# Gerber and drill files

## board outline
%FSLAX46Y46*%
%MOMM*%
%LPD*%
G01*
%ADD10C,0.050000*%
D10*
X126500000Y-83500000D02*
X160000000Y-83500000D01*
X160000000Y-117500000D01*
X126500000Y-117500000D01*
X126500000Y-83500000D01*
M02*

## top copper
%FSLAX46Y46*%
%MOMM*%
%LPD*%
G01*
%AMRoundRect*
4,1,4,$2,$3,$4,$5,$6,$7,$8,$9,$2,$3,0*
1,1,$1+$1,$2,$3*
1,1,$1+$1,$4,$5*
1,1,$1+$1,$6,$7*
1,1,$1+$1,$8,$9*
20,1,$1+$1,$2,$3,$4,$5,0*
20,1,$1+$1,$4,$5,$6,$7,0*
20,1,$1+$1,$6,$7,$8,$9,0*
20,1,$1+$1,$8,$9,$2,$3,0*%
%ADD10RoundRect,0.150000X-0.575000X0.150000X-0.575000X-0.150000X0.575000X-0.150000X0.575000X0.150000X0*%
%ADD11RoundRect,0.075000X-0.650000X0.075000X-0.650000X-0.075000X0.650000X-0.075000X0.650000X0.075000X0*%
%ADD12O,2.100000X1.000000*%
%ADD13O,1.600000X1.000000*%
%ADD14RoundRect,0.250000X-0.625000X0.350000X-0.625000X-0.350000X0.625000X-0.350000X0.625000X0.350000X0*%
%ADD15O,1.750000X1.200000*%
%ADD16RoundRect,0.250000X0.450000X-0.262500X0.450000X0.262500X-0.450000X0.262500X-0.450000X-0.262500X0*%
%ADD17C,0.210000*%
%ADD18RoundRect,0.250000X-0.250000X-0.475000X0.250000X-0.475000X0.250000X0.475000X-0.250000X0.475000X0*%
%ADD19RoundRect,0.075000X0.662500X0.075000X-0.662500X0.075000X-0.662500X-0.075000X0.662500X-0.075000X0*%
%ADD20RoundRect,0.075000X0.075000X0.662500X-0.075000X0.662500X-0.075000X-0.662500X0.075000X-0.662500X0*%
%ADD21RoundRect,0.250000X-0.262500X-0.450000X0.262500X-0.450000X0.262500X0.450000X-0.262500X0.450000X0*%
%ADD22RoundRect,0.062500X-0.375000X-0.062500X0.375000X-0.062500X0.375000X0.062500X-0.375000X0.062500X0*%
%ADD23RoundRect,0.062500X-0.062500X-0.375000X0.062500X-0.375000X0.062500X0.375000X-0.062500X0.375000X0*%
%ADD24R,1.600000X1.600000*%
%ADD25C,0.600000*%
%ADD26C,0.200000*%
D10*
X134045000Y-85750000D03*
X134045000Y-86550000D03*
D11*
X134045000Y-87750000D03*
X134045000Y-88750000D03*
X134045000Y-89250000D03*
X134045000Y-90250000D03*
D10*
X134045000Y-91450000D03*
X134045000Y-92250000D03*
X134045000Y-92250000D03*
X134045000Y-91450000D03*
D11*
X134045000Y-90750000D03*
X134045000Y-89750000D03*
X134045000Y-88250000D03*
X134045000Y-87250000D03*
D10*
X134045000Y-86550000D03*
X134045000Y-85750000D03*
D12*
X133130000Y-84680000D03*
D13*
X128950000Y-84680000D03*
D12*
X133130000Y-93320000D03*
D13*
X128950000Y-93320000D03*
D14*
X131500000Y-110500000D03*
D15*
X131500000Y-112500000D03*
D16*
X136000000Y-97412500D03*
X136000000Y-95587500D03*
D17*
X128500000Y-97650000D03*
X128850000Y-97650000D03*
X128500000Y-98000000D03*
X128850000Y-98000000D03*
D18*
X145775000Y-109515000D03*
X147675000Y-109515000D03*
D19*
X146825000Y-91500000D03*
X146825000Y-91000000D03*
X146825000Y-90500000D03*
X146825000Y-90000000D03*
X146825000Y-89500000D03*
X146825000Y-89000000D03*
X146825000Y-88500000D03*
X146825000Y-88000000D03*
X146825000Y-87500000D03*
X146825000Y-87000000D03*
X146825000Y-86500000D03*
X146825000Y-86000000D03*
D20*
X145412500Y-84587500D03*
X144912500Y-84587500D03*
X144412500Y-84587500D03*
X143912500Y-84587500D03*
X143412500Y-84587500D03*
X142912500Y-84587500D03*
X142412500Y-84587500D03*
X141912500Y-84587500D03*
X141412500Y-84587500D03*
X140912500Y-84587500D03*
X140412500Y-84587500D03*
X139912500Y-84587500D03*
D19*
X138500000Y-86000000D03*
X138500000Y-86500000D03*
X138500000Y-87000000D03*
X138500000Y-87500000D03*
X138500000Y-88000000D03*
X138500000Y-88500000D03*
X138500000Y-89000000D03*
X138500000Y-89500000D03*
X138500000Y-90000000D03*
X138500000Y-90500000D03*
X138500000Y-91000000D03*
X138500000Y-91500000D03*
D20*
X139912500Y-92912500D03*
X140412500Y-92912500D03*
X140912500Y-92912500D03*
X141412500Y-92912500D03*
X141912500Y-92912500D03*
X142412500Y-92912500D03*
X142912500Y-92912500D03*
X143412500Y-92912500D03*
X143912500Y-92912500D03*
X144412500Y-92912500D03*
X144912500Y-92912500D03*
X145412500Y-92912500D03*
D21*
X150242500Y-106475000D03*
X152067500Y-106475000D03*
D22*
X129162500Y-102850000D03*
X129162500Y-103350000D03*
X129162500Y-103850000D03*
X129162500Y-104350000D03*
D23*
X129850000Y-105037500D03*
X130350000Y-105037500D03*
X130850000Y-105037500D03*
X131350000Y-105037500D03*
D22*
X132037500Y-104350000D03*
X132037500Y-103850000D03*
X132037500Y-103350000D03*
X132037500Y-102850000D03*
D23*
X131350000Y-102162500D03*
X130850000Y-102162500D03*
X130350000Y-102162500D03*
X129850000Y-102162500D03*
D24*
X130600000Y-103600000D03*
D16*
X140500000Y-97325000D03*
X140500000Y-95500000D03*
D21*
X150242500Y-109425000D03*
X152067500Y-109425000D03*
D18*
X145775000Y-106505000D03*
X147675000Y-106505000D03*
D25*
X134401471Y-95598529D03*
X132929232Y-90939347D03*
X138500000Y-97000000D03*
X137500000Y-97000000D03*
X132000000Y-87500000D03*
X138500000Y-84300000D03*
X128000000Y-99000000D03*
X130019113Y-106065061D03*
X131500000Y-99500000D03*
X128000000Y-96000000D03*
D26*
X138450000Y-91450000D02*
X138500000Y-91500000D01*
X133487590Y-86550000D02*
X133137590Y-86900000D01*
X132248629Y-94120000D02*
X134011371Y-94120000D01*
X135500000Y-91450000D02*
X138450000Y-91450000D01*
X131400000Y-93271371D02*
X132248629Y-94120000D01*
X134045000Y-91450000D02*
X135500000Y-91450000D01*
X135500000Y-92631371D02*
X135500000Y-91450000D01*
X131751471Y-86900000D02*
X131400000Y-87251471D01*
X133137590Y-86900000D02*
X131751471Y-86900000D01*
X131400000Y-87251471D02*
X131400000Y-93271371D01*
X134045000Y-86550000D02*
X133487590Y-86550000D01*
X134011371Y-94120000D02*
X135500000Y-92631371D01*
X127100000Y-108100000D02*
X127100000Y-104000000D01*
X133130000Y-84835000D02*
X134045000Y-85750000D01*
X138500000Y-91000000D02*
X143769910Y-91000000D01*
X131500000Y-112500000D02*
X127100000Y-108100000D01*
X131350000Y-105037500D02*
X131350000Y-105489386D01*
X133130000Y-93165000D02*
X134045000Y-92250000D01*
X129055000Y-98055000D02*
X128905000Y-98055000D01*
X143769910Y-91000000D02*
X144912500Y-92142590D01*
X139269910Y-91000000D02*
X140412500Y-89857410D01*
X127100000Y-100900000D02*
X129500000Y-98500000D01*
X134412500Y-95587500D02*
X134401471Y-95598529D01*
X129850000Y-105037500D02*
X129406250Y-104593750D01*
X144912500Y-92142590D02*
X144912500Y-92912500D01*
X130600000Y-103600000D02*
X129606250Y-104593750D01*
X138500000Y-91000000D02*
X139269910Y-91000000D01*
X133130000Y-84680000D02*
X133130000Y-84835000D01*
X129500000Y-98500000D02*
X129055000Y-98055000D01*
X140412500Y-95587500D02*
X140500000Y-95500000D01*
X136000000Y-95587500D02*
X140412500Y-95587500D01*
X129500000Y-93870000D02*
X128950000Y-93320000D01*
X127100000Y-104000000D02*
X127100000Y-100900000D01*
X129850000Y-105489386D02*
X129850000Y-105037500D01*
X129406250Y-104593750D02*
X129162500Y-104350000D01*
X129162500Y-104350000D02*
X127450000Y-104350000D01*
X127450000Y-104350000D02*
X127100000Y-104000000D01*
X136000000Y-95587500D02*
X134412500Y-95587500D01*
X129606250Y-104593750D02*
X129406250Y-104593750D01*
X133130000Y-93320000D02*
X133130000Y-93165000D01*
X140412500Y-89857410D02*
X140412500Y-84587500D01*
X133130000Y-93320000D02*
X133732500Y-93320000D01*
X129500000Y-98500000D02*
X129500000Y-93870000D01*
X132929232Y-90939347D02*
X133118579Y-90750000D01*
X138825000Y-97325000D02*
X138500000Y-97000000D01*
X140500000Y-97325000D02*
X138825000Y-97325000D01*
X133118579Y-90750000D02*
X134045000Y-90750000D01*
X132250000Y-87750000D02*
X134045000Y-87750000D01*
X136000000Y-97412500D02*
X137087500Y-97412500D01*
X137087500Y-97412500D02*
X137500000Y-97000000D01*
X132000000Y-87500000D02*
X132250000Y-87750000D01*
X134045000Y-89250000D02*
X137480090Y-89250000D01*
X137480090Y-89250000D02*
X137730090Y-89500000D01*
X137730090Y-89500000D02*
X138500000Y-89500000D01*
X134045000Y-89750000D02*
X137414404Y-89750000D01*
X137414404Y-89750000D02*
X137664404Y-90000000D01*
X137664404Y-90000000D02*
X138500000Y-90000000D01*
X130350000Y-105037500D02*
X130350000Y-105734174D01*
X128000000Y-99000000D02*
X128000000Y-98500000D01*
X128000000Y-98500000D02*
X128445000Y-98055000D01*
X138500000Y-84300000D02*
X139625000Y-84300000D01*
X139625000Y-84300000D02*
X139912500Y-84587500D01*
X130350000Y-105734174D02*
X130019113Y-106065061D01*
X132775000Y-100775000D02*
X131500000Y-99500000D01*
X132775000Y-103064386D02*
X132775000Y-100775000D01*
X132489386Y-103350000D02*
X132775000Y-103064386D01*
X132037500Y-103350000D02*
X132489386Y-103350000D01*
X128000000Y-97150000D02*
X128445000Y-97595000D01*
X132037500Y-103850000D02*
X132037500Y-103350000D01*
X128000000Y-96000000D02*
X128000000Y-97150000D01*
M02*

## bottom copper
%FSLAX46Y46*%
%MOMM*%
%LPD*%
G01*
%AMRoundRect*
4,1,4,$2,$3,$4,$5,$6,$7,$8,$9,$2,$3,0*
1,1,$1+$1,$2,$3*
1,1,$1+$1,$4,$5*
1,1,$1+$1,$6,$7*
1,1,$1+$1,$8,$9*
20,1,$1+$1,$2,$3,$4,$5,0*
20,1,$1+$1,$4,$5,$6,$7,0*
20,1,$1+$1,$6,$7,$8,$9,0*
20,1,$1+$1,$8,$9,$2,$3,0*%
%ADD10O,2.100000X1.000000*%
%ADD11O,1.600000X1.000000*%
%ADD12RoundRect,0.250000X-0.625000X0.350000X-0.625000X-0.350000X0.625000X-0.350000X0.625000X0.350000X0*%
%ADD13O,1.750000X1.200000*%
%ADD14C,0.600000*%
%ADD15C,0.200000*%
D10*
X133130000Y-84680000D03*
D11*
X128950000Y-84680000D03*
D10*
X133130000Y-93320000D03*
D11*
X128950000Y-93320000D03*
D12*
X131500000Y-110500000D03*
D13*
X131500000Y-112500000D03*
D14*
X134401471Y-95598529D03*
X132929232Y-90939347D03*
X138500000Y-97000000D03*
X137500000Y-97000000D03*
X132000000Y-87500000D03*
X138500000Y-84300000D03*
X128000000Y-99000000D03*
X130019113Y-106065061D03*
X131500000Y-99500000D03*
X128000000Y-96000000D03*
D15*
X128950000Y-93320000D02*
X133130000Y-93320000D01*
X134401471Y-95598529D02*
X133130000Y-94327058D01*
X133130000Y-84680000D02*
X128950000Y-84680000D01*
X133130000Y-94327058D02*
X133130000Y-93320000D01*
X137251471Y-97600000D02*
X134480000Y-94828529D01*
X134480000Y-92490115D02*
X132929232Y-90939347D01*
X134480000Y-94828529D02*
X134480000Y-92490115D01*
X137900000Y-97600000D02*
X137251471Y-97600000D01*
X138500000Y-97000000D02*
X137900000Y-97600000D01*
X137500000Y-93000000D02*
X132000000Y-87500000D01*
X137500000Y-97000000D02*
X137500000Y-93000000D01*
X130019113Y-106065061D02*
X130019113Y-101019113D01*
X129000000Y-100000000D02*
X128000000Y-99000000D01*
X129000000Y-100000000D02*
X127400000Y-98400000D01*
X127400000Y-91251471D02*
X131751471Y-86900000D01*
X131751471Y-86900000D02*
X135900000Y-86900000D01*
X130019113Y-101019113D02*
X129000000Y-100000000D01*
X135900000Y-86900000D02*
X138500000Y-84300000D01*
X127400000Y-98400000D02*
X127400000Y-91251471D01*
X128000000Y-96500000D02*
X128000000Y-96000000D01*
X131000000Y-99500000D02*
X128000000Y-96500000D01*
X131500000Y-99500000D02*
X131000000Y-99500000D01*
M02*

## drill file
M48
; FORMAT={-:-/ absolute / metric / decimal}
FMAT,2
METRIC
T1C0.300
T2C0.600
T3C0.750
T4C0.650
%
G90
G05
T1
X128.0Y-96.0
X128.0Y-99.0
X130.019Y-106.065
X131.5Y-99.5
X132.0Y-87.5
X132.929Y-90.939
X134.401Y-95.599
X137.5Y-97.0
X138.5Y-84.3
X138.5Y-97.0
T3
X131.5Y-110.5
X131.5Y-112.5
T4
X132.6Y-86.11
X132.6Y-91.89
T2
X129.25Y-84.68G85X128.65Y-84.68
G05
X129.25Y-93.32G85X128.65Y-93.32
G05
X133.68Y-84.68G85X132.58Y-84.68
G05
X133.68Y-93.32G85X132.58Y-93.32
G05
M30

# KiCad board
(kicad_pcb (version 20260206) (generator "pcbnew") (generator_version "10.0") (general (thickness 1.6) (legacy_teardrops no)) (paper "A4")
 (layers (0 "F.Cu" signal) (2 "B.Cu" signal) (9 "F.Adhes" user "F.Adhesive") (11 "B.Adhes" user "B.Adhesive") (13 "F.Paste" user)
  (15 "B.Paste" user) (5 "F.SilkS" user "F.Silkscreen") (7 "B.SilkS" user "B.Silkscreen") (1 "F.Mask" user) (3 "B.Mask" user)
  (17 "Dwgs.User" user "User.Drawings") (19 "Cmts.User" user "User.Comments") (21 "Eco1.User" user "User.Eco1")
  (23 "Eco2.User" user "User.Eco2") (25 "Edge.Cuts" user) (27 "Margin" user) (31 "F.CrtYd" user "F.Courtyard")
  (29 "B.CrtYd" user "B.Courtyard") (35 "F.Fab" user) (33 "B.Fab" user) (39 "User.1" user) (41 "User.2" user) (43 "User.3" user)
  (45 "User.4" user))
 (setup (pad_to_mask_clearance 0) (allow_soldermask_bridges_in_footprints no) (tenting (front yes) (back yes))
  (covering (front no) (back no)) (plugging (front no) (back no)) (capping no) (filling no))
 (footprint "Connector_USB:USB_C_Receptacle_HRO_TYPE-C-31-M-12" (layer "F.Cu") (at 130 89 -90)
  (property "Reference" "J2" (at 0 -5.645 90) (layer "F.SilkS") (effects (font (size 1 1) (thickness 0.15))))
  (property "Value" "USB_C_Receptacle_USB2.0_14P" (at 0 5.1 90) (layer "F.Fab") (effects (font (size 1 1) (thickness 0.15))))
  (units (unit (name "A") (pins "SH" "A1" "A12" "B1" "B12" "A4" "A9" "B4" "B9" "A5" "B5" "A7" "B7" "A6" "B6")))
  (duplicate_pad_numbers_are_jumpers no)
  (pad "" np_thru_hole circle (at -2.89 -2.6 270) (size 0.65 0.65) (drill 0.65) (layers "*.Cu" "*.Mask"))
  (pad "" np_thru_hole circle (at 2.89 -2.6 270) (size 0.65 0.65) (drill 0.65) (layers "*.Cu" "*.Mask"))
  (pad "A1" smd roundrect (at -3.25 -4.045 270) (size 0.6 1.45) (layers "F.Cu" "F.Mask" "F.Paste") (roundrect_rratio 0.25) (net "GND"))
  (pad "A4" smd roundrect (at -2.45 -4.045 270) (size 0.6 1.45) (layers "F.Cu" "F.Mask" "F.Paste") (roundrect_rratio 0.25)
   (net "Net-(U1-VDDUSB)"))
  (pad "A5" smd roundrect (at -1.25 -4.045 270) (size 0.3 1.45) (layers "F.Cu" "F.Mask" "F.Paste") (roundrect_rratio 0.25)
   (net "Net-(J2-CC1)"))
  (pad "A6" smd roundrect (at -0.25 -4.045 270) (size 0.3 1.45) (layers "F.Cu" "F.Mask" "F.Paste") (roundrect_rratio 0.25)
   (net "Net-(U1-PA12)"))
  (pad "A7" smd roundrect (at 0.25 -4.045 270) (size 0.3 1.45) (layers "F.Cu" "F.Mask" "F.Paste") (roundrect_rratio 0.25)
   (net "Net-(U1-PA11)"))
  (pad "A8" smd roundrect (at 1.25 -4.045 270) (size 0.3 1.45) (layers "F.Cu" "F.Mask" "F.Paste") (roundrect_rratio 0.25))
  (pad "A9" smd roundrect (at 2.45 -4.045 270) (size 0.6 1.45) (layers "F.Cu" "F.Mask" "F.Paste") (roundrect_rratio 0.25)
   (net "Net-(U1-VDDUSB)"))
  (pad "A12" smd roundrect (at 3.25 -4.045 270) (size 0.6 1.45) (layers "F.Cu" "F.Mask" "F.Paste") (roundrect_rratio 0.25) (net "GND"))
  (pad "B1" smd roundrect (at 3.25 -4.045 270) (size 0.6 1.45) (layers "F.Cu" "F.Mask" "F.Paste") (roundrect_rratio 0.25) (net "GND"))
  (pad "B4" smd roundrect (at 2.45 -4.045 270) (size 0.6 1.45) (layers "F.Cu" "F.Mask" "F.Paste") (roundrect_rratio 0.25)
   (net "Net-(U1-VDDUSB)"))
  (pad "B5" smd roundrect (at 1.75 -4.045 270) (size 0.3 1.45) (layers "F.Cu" "F.Mask" "F.Paste") (roundrect_rratio 0.25)
   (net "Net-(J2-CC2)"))
  (pad "B6" smd roundrect (at 0.75 -4.045 270) (size 0.3 1.45) (layers "F.Cu" "F.Mask" "F.Paste") (roundrect_rratio 0.25)
   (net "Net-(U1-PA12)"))
  (pad "B7" smd roundrect (at -0.75 -4.045 270) (size 0.3 1.45) (layers "F.Cu" "F.Mask" "F.Paste") (roundrect_rratio 0.25)
   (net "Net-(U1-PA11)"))
  (pad "B8" smd roundrect (at -1.75 -4.045 270) (size 0.3 1.45) (layers "F.Cu" "F.Mask" "F.Paste") (roundrect_rratio 0.25))
  (pad "B9" smd roundrect (at -2.45 -4.045 270) (size 0.6 1.45) (layers "F.Cu" "F.Mask" "F.Paste") (roundrect_rratio 0.25)
   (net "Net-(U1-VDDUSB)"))
  (pad "B12" smd roundrect (at -3.25 -4.045 270) (size 0.6 1.45) (layers "F.Cu" "F.Mask" "F.Paste") (roundrect_rratio 0.25) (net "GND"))
  (pad "SH" thru_hole oval (at -4.32 -3.13 270) (size 1 2.1) (drill oval 0.6 1.7) (layers "*.Cu" "*.Mask") (remove_unused_layers no)
   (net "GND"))
  (pad "SH" thru_hole oval (at -4.32 1.05 270) (size 1 1.6) (drill oval 0.6 1.2) (layers "*.Cu" "*.Mask") (remove_unused_layers no)
   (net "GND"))
  (pad "SH" thru_hole oval (at 4.32 -3.13 270) (size 1 2.1) (drill oval 0.6 1.7) (layers "*.Cu" "*.Mask") (remove_unused_layers no)
   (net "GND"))
  (pad "SH" thru_hole oval (at 4.32 1.05 270) (size 1 1.6) (drill oval 0.6 1.2) (layers "*.Cu" "*.Mask") (remove_unused_layers no)
   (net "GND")))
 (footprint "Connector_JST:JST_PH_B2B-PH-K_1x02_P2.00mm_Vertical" (layer "F.Cu") (at 131.5 110.5 -90)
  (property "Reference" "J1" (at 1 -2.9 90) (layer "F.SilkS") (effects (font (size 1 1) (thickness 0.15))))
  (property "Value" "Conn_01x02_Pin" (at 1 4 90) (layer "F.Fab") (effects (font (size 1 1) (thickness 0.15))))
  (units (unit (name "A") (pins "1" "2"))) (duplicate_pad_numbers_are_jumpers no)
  (pad "1" thru_hole roundrect (at 0 0 270) (size 1.2 1.75) (drill 0.75) (layers "*.Cu" "*.Mask") (remove_unused_layers no)
   (roundrect_rratio 0.208333) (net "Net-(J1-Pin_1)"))
  (pad "2" thru_hole oval (at 2 0 270) (size 1.2 1.75) (drill 0.75) (layers "*.Cu" "*.Mask") (remove_unused_layers no) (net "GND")))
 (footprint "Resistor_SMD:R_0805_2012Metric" (layer "F.Cu") (at 136 96.5 90)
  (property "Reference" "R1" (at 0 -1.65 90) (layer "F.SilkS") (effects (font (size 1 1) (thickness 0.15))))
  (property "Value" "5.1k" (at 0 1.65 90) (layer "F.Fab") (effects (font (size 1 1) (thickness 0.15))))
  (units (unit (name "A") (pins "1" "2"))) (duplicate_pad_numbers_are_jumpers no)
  (pad "1" smd roundrect (at -0.9125 0 90) (size 1.025 1.4) (layers "F.Cu" "F.Mask" "F.Paste") (roundrect_rratio 0.243902)
   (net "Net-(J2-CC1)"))
  (pad "2" smd roundrect (at 0.9125 0 90) (size 1.025 1.4) (layers "F.Cu" "F.Mask" "F.Paste") (roundrect_rratio 0.243902) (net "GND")))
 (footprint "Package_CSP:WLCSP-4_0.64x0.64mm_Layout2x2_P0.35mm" (layer "F.Cu") (at 128.675 97.825)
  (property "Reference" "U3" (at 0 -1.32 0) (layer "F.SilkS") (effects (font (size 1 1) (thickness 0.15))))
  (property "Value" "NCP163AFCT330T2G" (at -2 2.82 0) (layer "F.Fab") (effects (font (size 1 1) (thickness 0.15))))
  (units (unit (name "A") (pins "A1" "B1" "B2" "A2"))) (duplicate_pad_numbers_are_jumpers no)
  (pad "A1" smd circle (at -0.175 -0.175) (size 0.21 0.21) (layers "F.Cu" "F.Mask" "F.Paste") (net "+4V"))
  (pad "A2" smd circle (at 0.175 -0.175) (size 0.21 0.21) (layers "F.Cu" "F.Mask" "F.Paste") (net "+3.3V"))
  (pad "B1" smd circle (at -0.175 0.175) (size 0.21 0.21) (layers "F.Cu" "F.Mask" "F.Paste") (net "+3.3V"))
  (pad "B2" smd circle (at 0.175 0.175) (size 0.21 0.21) (layers "F.Cu" "F.Mask" "F.Paste") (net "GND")))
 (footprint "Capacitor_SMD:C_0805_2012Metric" (layer "F.Cu") (at 146.725 109.515)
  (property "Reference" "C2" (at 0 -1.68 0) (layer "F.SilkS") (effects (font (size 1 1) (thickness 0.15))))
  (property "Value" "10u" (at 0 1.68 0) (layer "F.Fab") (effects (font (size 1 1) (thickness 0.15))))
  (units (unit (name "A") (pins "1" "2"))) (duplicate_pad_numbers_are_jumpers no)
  (pad "1" smd roundrect (at -0.95 0) (size 1 1.45) (layers "F.Cu" "F.Mask" "F.Paste") (roundrect_rratio 0.25) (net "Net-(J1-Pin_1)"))
  (pad "2" smd roundrect (at 0.95 0) (size 1 1.45) (layers "F.Cu" "F.Mask" "F.Paste") (roundrect_rratio 0.25) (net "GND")))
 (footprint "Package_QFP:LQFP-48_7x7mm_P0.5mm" (layer "F.Cu") (at 142.6625 88.75 180)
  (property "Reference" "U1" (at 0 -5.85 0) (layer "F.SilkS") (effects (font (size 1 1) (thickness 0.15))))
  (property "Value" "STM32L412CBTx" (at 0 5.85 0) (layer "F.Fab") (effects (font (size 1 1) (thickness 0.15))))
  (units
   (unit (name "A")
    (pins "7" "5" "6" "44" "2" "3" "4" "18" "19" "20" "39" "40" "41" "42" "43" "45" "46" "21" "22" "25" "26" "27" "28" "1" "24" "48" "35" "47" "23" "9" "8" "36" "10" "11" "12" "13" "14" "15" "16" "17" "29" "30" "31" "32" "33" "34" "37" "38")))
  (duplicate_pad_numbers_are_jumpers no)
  (pad "1" smd roundrect (at -4.1625 -2.75 180) (size 1.475 0.3) (layers "F.Cu" "F.Mask" "F.Paste") (roundrect_rratio 0.25) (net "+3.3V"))
  (pad "2" smd roundrect (at -4.1625 -2.25 180) (size 1.475 0.3) (layers "F.Cu" "F.Mask" "F.Paste") (roundrect_rratio 0.25)
   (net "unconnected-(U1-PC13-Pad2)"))
  (pad "3" smd roundrect (at -4.1625 -1.75 180) (size 1.475 0.3) (layers "F.Cu" "F.Mask" "F.Paste") (roundrect_rratio 0.25)
   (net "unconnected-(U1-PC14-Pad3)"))
  (pad "4" smd roundrect (at -4.1625 -1.25 180) (size 1.475 0.3) (layers "F.Cu" "F.Mask" "F.Paste") (roundrect_rratio 0.25)
   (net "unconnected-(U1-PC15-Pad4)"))
  (pad "5" smd roundrect (at -4.1625 -0.75 180) (size 1.475 0.3) (layers "F.Cu" "F.Mask" "F.Paste") (roundrect_rratio 0.25)
   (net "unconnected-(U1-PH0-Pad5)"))
  (pad "6" smd roundrect (at -4.1625 -0.25 180) (size 1.475 0.3) (layers "F.Cu" "F.Mask" "F.Paste") (roundrect_rratio 0.25)
   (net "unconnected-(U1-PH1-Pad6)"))
  (pad "7" smd roundrect (at -4.1625 0.25 180) (size 1.475 0.3) (layers "F.Cu" "F.Mask" "F.Paste") (roundrect_rratio 0.25)
   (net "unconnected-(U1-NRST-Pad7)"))
  (pad "8" smd roundrect (at -4.1625 0.75 180) (size 1.475 0.3) (layers "F.Cu" "F.Mask" "F.Paste") (roundrect_rratio 0.25) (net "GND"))
  (pad "9" smd roundrect (at -4.1625 1.25 180) (size 1.475 0.3) (layers "F.Cu" "F.Mask" "F.Paste") (roundrect_rratio 0.25) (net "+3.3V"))
  (pad "10" smd roundrect (at -4.1625 1.75 180) (size 1.475 0.3) (layers "F.Cu" "F.Mask" "F.Paste") (roundrect_rratio 0.25)
   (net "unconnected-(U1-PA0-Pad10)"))
  (pad "11" smd roundrect (at -4.1625 2.25 180) (size 1.475 0.3) (layers "F.Cu" "F.Mask" "F.Paste") (roundrect_rratio 0.25)
   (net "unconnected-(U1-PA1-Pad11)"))
  (pad "12" smd roundrect (at -4.1625 2.75 180) (size 1.475 0.3) (layers "F.Cu" "F.Mask" "F.Paste") (roundrect_rratio 0.25)
   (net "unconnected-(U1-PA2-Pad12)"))
  (pad "13" smd roundrect (at -2.75 4.1625 180) (size 0.3 1.475) (layers "F.Cu" "F.Mask" "F.Paste") (roundrect_rratio 0.25)
   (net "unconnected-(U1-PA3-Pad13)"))
  (pad "14" smd roundrect (at -2.25 4.1625 180) (size 0.3 1.475) (layers "F.Cu" "F.Mask" "F.Paste") (roundrect_rratio 0.25)
   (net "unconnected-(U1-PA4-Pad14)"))
  (pad "15" smd roundrect (at -1.75 4.1625 180) (size 0.3 1.475) (layers "F.Cu" "F.Mask" "F.Paste") (roundrect_rratio 0.25)
   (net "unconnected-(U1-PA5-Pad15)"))
  (pad "16" smd roundrect (at -1.25 4.1625 180) (size 0.3 1.475) (layers "F.Cu" "F.Mask" "F.Paste") (roundrect_rratio 0.25)
   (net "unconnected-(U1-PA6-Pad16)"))
  (pad "17" smd roundrect (at -0.75 4.1625 180) (size 0.3 1.475) (layers "F.Cu" "F.Mask" "F.Paste") (roundrect_rratio 0.25)
   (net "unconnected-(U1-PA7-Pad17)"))
  (pad "18" smd roundrect (at -0.25 4.1625 180) (size 0.3 1.475) (layers "F.Cu" "F.Mask" "F.Paste") (roundrect_rratio 0.25)
   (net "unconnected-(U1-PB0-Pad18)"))
  (pad "19" smd roundrect (at 0.25 4.1625 180) (size 0.3 1.475) (layers "F.Cu" "F.Mask" "F.Paste") (roundrect_rratio 0.25)
   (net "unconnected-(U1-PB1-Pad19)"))
  (pad "20" smd roundrect (at 0.75 4.1625 180) (size 0.3 1.475) (layers "F.Cu" "F.Mask" "F.Paste") (roundrect_rratio 0.25)
   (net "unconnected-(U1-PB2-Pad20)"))
  (pad "21" smd roundrect (at 1.25 4.1625 180) (size 0.3 1.475) (layers "F.Cu" "F.Mask" "F.Paste") (roundrect_rratio 0.25)
   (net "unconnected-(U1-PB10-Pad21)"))
  (pad "22" smd roundrect (at 1.75 4.1625 180) (size 0.3 1.475) (layers "F.Cu" "F.Mask" "F.Paste") (roundrect_rratio 0.25)
   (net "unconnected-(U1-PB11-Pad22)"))
  (pad "23" smd roundrect (at 2.25 4.1625 180) (size 0.3 1.475) (layers "F.Cu" "F.Mask" "F.Paste") (roundrect_rratio 0.25) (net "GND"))
  (pad "24" smd roundrect (at 2.75 4.1625 180) (size 0.3 1.475) (layers "F.Cu" "F.Mask" "F.Paste") (roundrect_rratio 0.25) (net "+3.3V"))
  (pad "25" smd roundrect (at 4.1625 2.75 180) (size 1.475 0.3) (layers "F.Cu" "F.Mask" "F.Paste") (roundrect_rratio 0.25)
   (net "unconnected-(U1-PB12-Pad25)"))
  (pad "26" smd roundrect (at 4.1625 2.25 180) (size 1.475 0.3) (layers "F.Cu" "F.Mask" "F.Paste") (roundrect_rratio 0.25)
   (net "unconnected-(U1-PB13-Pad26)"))
  (pad "27" smd roundrect (at 4.1625 1.75 180) (size 1.475 0.3) (layers "F.Cu" "F.Mask" "F.Paste") (roundrect_rratio 0.25)
   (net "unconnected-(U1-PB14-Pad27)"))
  (pad "28" smd roundrect (at 4.1625 1.25 180) (size 1.475 0.3) (layers "F.Cu" "F.Mask" "F.Paste") (roundrect_rratio 0.25)
   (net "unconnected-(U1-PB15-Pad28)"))
  (pad "29" smd roundrect (at 4.1625 0.75 180) (size 1.475 0.3) (layers "F.Cu" "F.Mask" "F.Paste") (roundrect_rratio 0.25)
   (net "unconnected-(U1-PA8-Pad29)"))
  (pad "30" smd roundrect (at 4.1625 0.25 180) (size 1.475 0.3) (layers "F.Cu" "F.Mask" "F.Paste") (roundrect_rratio 0.25)
   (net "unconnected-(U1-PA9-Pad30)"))
  (pad "31" smd roundrect (at 4.1625 -0.25 180) (size 1.475 0.3) (layers "F.Cu" "F.Mask" "F.Paste") (roundrect_rratio 0.25)
   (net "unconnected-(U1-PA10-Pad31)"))
  (pad "32" smd roundrect (at 4.1625 -0.75 180) (size 1.475 0.3) (layers "F.Cu" "F.Mask" "F.Paste") (roundrect_rratio 0.25)
   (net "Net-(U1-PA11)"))
  (pad "33" smd roundrect (at 4.1625 -1.25 180) (size 1.475 0.3) (layers "F.Cu" "F.Mask" "F.Paste") (roundrect_rratio 0.25)
   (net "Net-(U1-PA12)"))
  (pad "34" smd roundrect (at 4.1625 -1.75 180) (size 1.475 0.3) (layers "F.Cu" "F.Mask" "F.Paste") (roundrect_rratio 0.25)
   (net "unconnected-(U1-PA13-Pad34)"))
  (pad "35" smd roundrect (at 4.1625 -2.25 180) (size 1.475 0.3) (layers "F.Cu" "F.Mask" "F.Paste") (roundrect_rratio 0.25) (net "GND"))
  (pad "36" smd roundrect (at 4.1625 -2.75 180) (size 1.475 0.3) (layers "F.Cu" "F.Mask" "F.Paste") (roundrect_rratio 0.25)
   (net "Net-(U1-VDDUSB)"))
  (pad "37" smd roundrect (at 2.75 -4.1625 180) (size 0.3 1.475) (layers "F.Cu" "F.Mask" "F.Paste") (roundrect_rratio 0.25)
   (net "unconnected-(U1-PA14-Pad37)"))
  (pad "38" smd roundrect (at 2.25 -4.1625 180) (size 0.3 1.475) (layers "F.Cu" "F.Mask" "F.Paste") (roundrect_rratio 0.25)
   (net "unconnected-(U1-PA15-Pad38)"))
  (pad "39" smd roundrect (at 1.75 -4.1625 180) (size 0.3 1.475) (layers "F.Cu" "F.Mask" "F.Paste") (roundrect_rratio 0.25)
   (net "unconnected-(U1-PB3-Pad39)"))
  (pad "40" smd roundrect (at 1.25 -4.1625 180) (size 0.3 1.475) (layers "F.Cu" "F.Mask" "F.Paste") (roundrect_rratio 0.25)
   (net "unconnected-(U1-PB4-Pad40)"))
  (pad "41" smd roundrect (at 0.75 -4.1625 180) (size 0.3 1.475) (layers "F.Cu" "F.Mask" "F.Paste") (roundrect_rratio 0.25)
   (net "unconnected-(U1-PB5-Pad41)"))
  (pad "42" smd roundrect (at 0.25 -4.1625 180) (size 0.3 1.475) (layers "F.Cu" "F.Mask" "F.Paste") (roundrect_rratio 0.25)
   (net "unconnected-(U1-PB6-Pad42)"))
  (pad "43" smd roundrect (at -0.25 -4.1625 180) (size 0.3 1.475) (layers "F.Cu" "F.Mask" "F.Paste") (roundrect_rratio 0.25)
   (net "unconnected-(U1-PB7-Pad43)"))
  (pad "44" smd roundrect (at -0.75 -4.1625 180) (size 0.3 1.475) (layers "F.Cu" "F.Mask" "F.Paste") (roundrect_rratio 0.25)
   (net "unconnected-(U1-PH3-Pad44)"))
  (pad "45" smd roundrect (at -1.25 -4.1625 180) (size 0.3 1.475) (layers "F.Cu" "F.Mask" "F.Paste") (roundrect_rratio 0.25)
   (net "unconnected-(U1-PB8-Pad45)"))
  (pad "46" smd roundrect (at -1.75 -4.1625 180) (size 0.3 1.475) (layers "F.Cu" "F.Mask" "F.Paste") (roundrect_rratio 0.25)
   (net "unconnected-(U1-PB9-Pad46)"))
  (pad "47" smd roundrect (at -2.25 -4.1625 180) (size 0.3 1.475) (layers "F.Cu" "F.Mask" "F.Paste") (roundrect_rratio 0.25) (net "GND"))
  (pad "48" smd roundrect (at -2.75 -4.1625 180) (size 0.3 1.475) (layers "F.Cu" "F.Mask" "F.Paste") (roundrect_rratio 0.25) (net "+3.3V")))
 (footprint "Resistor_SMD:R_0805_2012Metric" (layer "F.Cu") (at 151.155 106.475)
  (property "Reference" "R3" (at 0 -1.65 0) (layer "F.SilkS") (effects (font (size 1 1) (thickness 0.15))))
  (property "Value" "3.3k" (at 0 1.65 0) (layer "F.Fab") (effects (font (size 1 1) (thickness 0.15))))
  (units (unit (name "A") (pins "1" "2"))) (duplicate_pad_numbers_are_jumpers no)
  (pad "1" smd roundrect (at -0.9125 0) (size 1.025 1.4) (layers "F.Cu" "F.Mask" "F.Paste") (roundrect_rratio 0.243902)
   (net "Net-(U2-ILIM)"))
  (pad "2" smd roundrect (at 0.9125 0) (size 1.025 1.4) (layers "F.Cu" "F.Mask" "F.Paste") (roundrect_rratio 0.243902) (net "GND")))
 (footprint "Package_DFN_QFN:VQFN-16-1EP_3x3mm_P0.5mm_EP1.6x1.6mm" (layer "F.Cu") (at 130.6 103.6)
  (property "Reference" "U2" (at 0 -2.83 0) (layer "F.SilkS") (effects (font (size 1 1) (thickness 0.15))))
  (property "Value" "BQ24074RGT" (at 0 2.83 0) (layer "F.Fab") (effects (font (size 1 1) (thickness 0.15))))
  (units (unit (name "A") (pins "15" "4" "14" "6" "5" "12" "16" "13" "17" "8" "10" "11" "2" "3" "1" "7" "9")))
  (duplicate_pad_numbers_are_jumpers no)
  (pad "" smd roundrect (at -0.4 -0.4) (size 0.64 0.64) (layers "F.Paste") (roundrect_rratio 0.25))
  (pad "" smd roundrect (at -0.4 0.4) (size 0.64 0.64) (layers "F.Paste") (roundrect_rratio 0.25))
  (pad "" smd roundrect (at 0.4 -0.4) (size 0.64 0.64) (layers "F.Paste") (roundrect_rratio 0.25))
  (pad "" smd roundrect (at 0.4 0.4) (size 0.64 0.64) (layers "F.Paste") (roundrect_rratio 0.25))
  (pad "1" smd roundrect (at -1.4375 -0.75) (size 0.875 0.25) (layers "F.Cu" "F.Mask" "F.Paste") (roundrect_rratio 0.25) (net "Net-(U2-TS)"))
  (pad "2" smd roundrect (at -1.4375 -0.25) (size 0.875 0.25) (layers "F.Cu" "F.Mask" "F.Paste") (roundrect_rratio 0.25)
   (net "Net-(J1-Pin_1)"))
  (pad "3" smd roundrect (at -1.4375 0.25) (size 0.875 0.25) (layers "F.Cu" "F.Mask" "F.Paste") (roundrect_rratio 0.25)
   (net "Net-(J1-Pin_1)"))
  (pad "4" smd roundrect (at -1.4375 0.75) (size 0.875 0.25) (layers "F.Cu" "F.Mask" "F.Paste") (roundrect_rratio 0.25) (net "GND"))
  (pad "5" smd roundrect (at -0.75 1.4375) (size 0.25 0.875) (layers "F.Cu" "F.Mask" "F.Paste") (roundrect_rratio 0.25) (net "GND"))
  (pad "6" smd roundrect (at -0.25 1.4375) (size 0.25 0.875) (layers "F.Cu" "F.Mask" "F.Paste") (roundrect_rratio 0.25) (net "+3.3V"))
  (pad "7" smd roundrect (at 0.25 1.4375) (size 0.25 0.875) (layers "F.Cu" "F.Mask" "F.Paste") (roundrect_rratio 0.25)
   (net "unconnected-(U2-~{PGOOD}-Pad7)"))
  (pad "8" smd roundrect (at 0.75 1.4375) (size 0.25 0.875) (layers "F.Cu" "F.Mask" "F.Paste") (roundrect_rratio 0.25) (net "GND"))
  (pad "9" smd roundrect (at 1.4375 0.75) (size 0.875 0.25) (layers "F.Cu" "F.Mask" "F.Paste") (roundrect_rratio 0.25)
   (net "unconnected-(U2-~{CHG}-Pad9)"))
  (pad "10" smd roundrect (at 1.4375 0.25) (size 0.875 0.25) (layers "F.Cu" "F.Mask" "F.Paste") (roundrect_rratio 0.25) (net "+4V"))
  (pad "11" smd roundrect (at 1.4375 -0.25) (size 0.875 0.25) (layers "F.Cu" "F.Mask" "F.Paste") (roundrect_rratio 0.25) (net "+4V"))
  (pad "12" smd roundrect (at 1.4375 -0.75) (size 0.875 0.25) (layers "F.Cu" "F.Mask" "F.Paste") (roundrect_rratio 0.25)
   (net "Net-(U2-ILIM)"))
  (pad "13" smd roundrect (at 0.75 -1.4375) (size 0.25 0.875) (layers "F.Cu" "F.Mask" "F.Paste") (roundrect_rratio 0.25)
   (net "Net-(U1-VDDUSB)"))
  (pad "14" smd roundrect (at 0.25 -1.4375) (size 0.25 0.875) (layers "F.Cu" "F.Mask" "F.Paste") (roundrect_rratio 0.25)
   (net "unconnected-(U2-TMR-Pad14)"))
  (pad "15" smd roundrect (at -0.25 -1.4375) (size 0.25 0.875) (layers "F.Cu" "F.Mask" "F.Paste") (roundrect_rratio 0.25)
   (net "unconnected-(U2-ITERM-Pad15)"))
  (pad "16" smd roundrect (at -0.75 -1.4375) (size 0.25 0.875) (layers "F.Cu" "F.Mask" "F.Paste") (roundrect_rratio 0.25)
   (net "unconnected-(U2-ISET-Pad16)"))
  (pad "17" smd rect (at 0 0) (size 1.6 1.6) (layers "F.Cu" "F.Mask") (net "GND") (zone_connect 2)))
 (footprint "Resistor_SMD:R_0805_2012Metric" (layer "F.Cu") (at 140.5 96.4125 90)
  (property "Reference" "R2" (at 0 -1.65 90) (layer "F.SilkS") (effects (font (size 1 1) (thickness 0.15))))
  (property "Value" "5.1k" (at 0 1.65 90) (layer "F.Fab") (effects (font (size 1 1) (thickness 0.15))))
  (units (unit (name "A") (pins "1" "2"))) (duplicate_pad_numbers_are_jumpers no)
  (pad "1" smd roundrect (at -0.9125 0 90) (size 1.025 1.4) (layers "F.Cu" "F.Mask" "F.Paste") (roundrect_rratio 0.243902)
   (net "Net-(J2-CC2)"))
  (pad "2" smd roundrect (at 0.9125 0 90) (size 1.025 1.4) (layers "F.Cu" "F.Mask" "F.Paste") (roundrect_rratio 0.243902) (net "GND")))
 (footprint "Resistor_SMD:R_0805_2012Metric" (layer "F.Cu") (at 151.155 109.425)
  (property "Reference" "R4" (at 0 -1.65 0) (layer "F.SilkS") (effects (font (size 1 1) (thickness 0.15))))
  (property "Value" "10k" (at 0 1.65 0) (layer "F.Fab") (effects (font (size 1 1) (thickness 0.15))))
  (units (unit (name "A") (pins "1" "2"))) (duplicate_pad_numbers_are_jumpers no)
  (pad "1" smd roundrect (at -0.9125 0) (size 1.025 1.4) (layers "F.Cu" "F.Mask" "F.Paste") (roundrect_rratio 0.243902) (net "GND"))
  (pad "2" smd roundrect (at 0.9125 0) (size 1.025 1.4) (layers "F.Cu" "F.Mask" "F.Paste") (roundrect_rratio 0.243902) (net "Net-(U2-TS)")))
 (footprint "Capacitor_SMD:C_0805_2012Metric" (layer "F.Cu") (at 146.725 106.505)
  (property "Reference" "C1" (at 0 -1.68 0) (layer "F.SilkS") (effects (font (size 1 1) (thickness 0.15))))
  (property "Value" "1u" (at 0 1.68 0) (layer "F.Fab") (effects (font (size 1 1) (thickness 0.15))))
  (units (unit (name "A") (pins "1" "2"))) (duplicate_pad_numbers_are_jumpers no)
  (pad "1" smd roundrect (at -0.95 0) (size 1 1.45) (layers "F.Cu" "F.Mask" "F.Paste") (roundrect_rratio 0.25) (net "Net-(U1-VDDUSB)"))
  (pad "2" smd roundrect (at 0.95 0) (size 1 1.45) (layers "F.Cu" "F.Mask" "F.Paste") (roundrect_rratio 0.25) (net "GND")))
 (gr_rect (start 126.5 83.5) (end 160 117.5) (stroke (width 0.05) (type default)) (fill no) (layer "Edge.Cuts"))
 (segment (start 138.45 91.45) (end 138.5 91.5) (width 0.2) (layer "F.Cu") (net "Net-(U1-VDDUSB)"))
 (segment (start 133.48759 86.55) (end 133.13759 86.9) (width 0.2) (layer "F.Cu") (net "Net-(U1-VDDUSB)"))
 (segment (start 132.248629 94.12) (end 134.011371 94.12) (width 0.2) (layer "F.Cu") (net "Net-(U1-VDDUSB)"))
 (segment (start 135.5 91.45) (end 138.45 91.45) (width 0.2) (layer "F.Cu") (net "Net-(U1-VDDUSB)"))
 (segment (start 131.4 93.271371) (end 132.248629 94.12) (width 0.2) (layer "F.Cu") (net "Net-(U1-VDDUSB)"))
 (segment (start 134.045 91.45) (end 135.5 91.45) (width 0.2) (layer "F.Cu") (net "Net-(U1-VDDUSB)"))
 (segment (start 135.5 92.631371) (end 135.5 91.45) (width 0.2) (layer "F.Cu") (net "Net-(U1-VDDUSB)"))
 (segment (start 131.751471 86.9) (end 131.4 87.251471) (width 0.2) (layer "F.Cu") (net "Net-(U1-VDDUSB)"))
 (segment (start 133.13759 86.9) (end 131.751471 86.9) (width 0.2) (layer "F.Cu") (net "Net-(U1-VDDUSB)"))
 (segment (start 131.4 87.251471) (end 131.4 93.271371) (width 0.2) (layer "F.Cu") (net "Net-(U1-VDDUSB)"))
 (segment (start 134.045 86.55) (end 133.48759 86.55) (width 0.2) (layer "F.Cu") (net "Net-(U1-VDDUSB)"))
 (segment (start 134.011371 94.12) (end 135.5 92.631371) (width 0.2) (layer "F.Cu") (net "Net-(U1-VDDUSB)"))
 (segment (start 127.1 108.1) (end 127.1 104) (width 0.2) (layer "F.Cu") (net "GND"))
 (segment (start 133.13 84.835) (end 134.045 85.75) (width 0.2) (layer "F.Cu") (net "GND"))
 (segment (start 138.5 91) (end 143.76991 91) (width 0.2) (layer "F.Cu") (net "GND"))
 (segment (start 131.5 112.5) (end 127.1 108.1) (width 0.2) (layer "F.Cu") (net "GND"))
 (segment (start 131.35 105.0375) (end 131.35 105.489386) (width 0.2) (layer "F.Cu") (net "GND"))
 (segment (start 133.13 93.165) (end 134.045 92.25) (width 0.2) (layer "F.Cu") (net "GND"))
 (segment (start 129.055 98.055) (end 128.905 98.055) (width 0.2) (layer "F.Cu") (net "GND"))
 (segment (start 143.76991 91) (end 144.9125 92.14259) (width 0.2) (layer "F.Cu") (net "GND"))
 (segment (start 139.26991 91) (end 140.4125 89.85741) (width 0.2) (layer "F.Cu") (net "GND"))
 (segment (start 127.1 100.9) (end 129.5 98.5) (width 0.2) (layer "F.Cu") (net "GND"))
 (segment (start 134.4125 95.5875) (end 134.401471 95.598529) (width 0.2) (layer "F.Cu") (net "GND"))
 (segment (start 129.85 105.0375) (end 129.40625 104.59375) (width 0.2) (layer "F.Cu") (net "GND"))
 (segment (start 144.9125 92.14259) (end 144.9125 92.9125) (width 0.2) (layer "F.Cu") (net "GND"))
 (segment (start 130.6 103.6) (end 129.60625 104.59375) (width 0.2) (layer "F.Cu") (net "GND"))
 (segment (start 138.5 91) (end 139.26991 91) (width 0.2) (layer "F.Cu") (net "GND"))
 (segment (start 133.13 84.68) (end 133.13 84.835) (width 0.2) (layer "F.Cu") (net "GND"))
 (segment (start 129.5 98.5) (end 129.055 98.055) (width 0.2) (layer "F.Cu") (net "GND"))
 (segment (start 140.4125 95.5875) (end 140.5 95.5) (width 0.2) (layer "F.Cu") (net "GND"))
 (segment (start 136 95.5875) (end 140.4125 95.5875) (width 0.2) (layer "F.Cu") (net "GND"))
 (segment (start 129.5 93.87) (end 128.95 93.32) (width 0.2) (layer "F.Cu") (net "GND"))
 (segment (start 127.1 104) (end 127.1 100.9) (width 0.2) (layer "F.Cu") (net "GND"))
 (segment (start 129.85 105.489386) (end 129.85 105.0375) (width 0.2) (layer "F.Cu") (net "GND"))
 (segment (start 129.40625 104.59375) (end 129.1625 104.35) (width 0.2) (layer "F.Cu") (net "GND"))
 (segment (start 129.1625 104.35) (end 127.45 104.35) (width 0.2) (layer "F.Cu") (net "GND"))
 (segment (start 127.45 104.35) (end 127.1 104) (width 0.2) (layer "F.Cu") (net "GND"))
 (segment (start 136 95.5875) (end 134.4125 95.5875) (width 0.2) (layer "F.Cu") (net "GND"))
 (segment (start 129.60625 104.59375) (end 129.40625 104.59375) (width 0.2) (layer "F.Cu") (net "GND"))
 (segment (start 133.13 93.32) (end 133.13 93.165) (width 0.2) (layer "F.Cu") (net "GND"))
 (segment (start 140.4125 89.85741) (end 140.4125 84.5875) (width 0.2) (layer "F.Cu") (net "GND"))
 (segment (start 133.13 93.32) (end 133.7325 93.32) (width 0.2) (layer "F.Cu") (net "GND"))
 (segment (start 129.5 98.5) (end 129.5 93.87) (width 0.2) (layer "F.Cu") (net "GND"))
 (via (at 134.401471 95.598529) (size 0.6) (drill 0.3) (layers "F.Cu" "B.Cu") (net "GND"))
 (segment (start 128.95 93.32) (end 133.13 93.32) (width 0.2) (layer "B.Cu") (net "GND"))
 (segment (start 134.401471 95.598529) (end 133.13 94.327058) (width 0.2) (layer "B.Cu") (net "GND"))
 (segment (start 133.13 84.68) (end 128.95 84.68) (width 0.2) (layer "B.Cu") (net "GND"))
 (segment (start 133.13 94.327058) (end 133.13 93.32) (width 0.2) (layer "B.Cu") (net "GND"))
 (segment (start 132.929232 90.939347) (end 133.118579 90.75) (width 0.2) (layer "F.Cu") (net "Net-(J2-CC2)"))
 (segment (start 138.825 97.325) (end 138.5 97) (width 0.2) (layer "F.Cu") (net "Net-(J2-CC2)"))
 (segment (start 140.5 97.325) (end 138.825 97.325) (width 0.2) (layer "F.Cu") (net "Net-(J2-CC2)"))
 (segment (start 133.118579 90.75) (end 134.045 90.75) (width 0.2) (layer "F.Cu") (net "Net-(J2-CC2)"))
 (via (at 132.929232 90.939347) (size 0.6) (drill 0.3) (layers "F.Cu" "B.Cu") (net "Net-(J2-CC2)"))
 (via (at 138.5 97) (size 0.6) (drill 0.3) (layers "F.Cu" "B.Cu") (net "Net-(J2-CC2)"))
 (segment (start 137.251471 97.6) (end 134.48 94.828529) (width 0.2) (layer "B.Cu") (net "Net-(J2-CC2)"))
 (segment (start 134.48 92.490115) (end 132.929232 90.939347) (width 0.2) (layer "B.Cu") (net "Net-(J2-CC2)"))
 (segment (start 134.48 94.828529) (end 134.48 92.490115) (width 0.2) (layer "B.Cu") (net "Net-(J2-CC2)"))
 (segment (start 137.9 97.6) (end 137.251471 97.6) (width 0.2) (layer "B.Cu") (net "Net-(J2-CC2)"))
 (segment (start 138.5 97) (end 137.9 97.6) (width 0.2) (layer "B.Cu") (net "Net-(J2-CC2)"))
 (segment (start 132.25 87.75) (end 134.045 87.75) (width 0.2) (layer "F.Cu") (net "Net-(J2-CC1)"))
 (segment (start 136 97.4125) (end 137.0875 97.4125) (width 0.2) (layer "F.Cu") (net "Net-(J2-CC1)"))
 (segment (start 137.0875 97.4125) (end 137.5 97) (width 0.2) (layer "F.Cu") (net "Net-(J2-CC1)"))
 (segment (start 132 87.5) (end 132.25 87.75) (width 0.2) (layer "F.Cu") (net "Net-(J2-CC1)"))
 (via (at 137.5 97) (size 0.6) (drill 0.3) (layers "F.Cu" "B.Cu") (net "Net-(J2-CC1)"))
 (via (at 132 87.5) (size 0.6) (drill 0.3) (layers "F.Cu" "B.Cu") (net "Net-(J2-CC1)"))
 (segment (start 137.5 93) (end 132 87.5) (width 0.2) (layer "B.Cu") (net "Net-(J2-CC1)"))
 (segment (start 137.5 97) (end 137.5 93) (width 0.2) (layer "B.Cu") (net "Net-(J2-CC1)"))
 (segment (start 134.045 89.25) (end 137.48009 89.25) (width 0.2) (layer "F.Cu") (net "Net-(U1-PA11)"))
 (segment (start 137.48009 89.25) (end 137.73009 89.5) (width 0.2) (layer "F.Cu") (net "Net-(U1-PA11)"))
 (segment (start 137.73009 89.5) (end 138.5 89.5) (width 0.2) (layer "F.Cu") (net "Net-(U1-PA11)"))
 (segment (start 134.045 89.75) (end 137.414404 89.75) (width 0.2) (layer "F.Cu") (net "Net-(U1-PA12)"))
 (segment (start 137.414404 89.75) (end 137.664404 90) (width 0.2) (layer "F.Cu") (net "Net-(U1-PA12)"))
 (segment (start 137.664404 90) (end 138.5 90) (width 0.2) (layer "F.Cu") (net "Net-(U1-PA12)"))
 (segment (start 130.35 105.0375) (end 130.35 105.734174) (width 0.2) (layer "F.Cu") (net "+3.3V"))
 (segment (start 128 99) (end 128 98.5) (width 0.2) (layer "F.Cu") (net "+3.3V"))
 (segment (start 128 98.5) (end 128.445 98.055) (width 0.2) (layer "F.Cu") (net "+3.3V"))
 (segment (start 138.5 84.3) (end 139.625 84.3) (width 0.2) (layer "F.Cu") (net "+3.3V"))
 (segment (start 139.625 84.3) (end 139.9125 84.5875) (width 0.2) (layer "F.Cu") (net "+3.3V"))
 (segment (start 130.35 105.734174) (end 130.019113 106.065061) (width 0.2) (layer "F.Cu") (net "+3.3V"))
 (via (at 138.5 84.3) (size 0.6) (drill 0.3) (layers "F.Cu" "B.Cu") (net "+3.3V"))
 (via (at 128 99) (size 0.6) (drill 0.3) (layers "F.Cu" "B.Cu") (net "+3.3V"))
 (via (at 130.019113 106.065061) (size 0.6) (drill 0.3) (layers "F.Cu" "B.Cu") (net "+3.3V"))
 (segment (start 130.019113 106.065061) (end 130.019113 101.019113) (width 0.2) (layer "B.Cu") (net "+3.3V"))
 (segment (start 129 100) (end 128 99) (width 0.2) (layer "B.Cu") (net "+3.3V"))
 (segment (start 129 100) (end 127.4 98.4) (width 0.2) (layer "B.Cu") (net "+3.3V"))
 (segment (start 127.4 91.251471) (end 131.751471 86.9) (width 0.2) (layer "B.Cu") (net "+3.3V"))
 (segment (start 131.751471 86.9) (end 135.9 86.9) (width 0.2) (layer "B.Cu") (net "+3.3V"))
 (segment (start 130.019113 101.019113) (end 129 100) (width 0.2) (layer "B.Cu") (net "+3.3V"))
 (segment (start 135.9 86.9) (end 138.5 84.3) (width 0.2) (layer "B.Cu") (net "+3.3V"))
 (segment (start 127.4 98.4) (end 127.4 91.251471) (width 0.2) (layer "B.Cu") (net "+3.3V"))
 (segment (start 132.775 100.775) (end 131.5 99.5) (width 0.2) (layer "F.Cu") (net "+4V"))
 (segment (start 132.775 103.064386) (end 132.775 100.775) (width 0.2) (layer "F.Cu") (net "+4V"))
 (segment (start 132.489386 103.35) (end 132.775 103.064386) (width 0.2) (layer "F.Cu") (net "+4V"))
 (segment (start 132.0375 103.35) (end 132.489386 103.35) (width 0.2) (layer "F.Cu") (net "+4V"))
 (segment (start 128 97.15) (end 128.445 97.595) (width 0.2) (layer "F.Cu") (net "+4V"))
 (segment (start 132.0375 103.85) (end 132.0375 103.35) (width 0.2) (layer "F.Cu") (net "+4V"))
 (segment (start 128 96) (end 128 97.15) (width 0.2) (layer "F.Cu") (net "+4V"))
 (via (at 131.5 99.5) (size 0.6) (drill 0.3) (layers "F.Cu" "B.Cu") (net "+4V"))
 (via (at 128 96) (size 0.6) (drill 0.3) (layers "F.Cu" "B.Cu") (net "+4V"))
 (segment (start 128 96.5) (end 128 96) (width 0.2) (layer "B.Cu") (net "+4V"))
 (segment (start 131 99.5) (end 128 96.5) (width 0.2) (layer "B.Cu") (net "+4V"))
 (segment (start 131.5 99.5) (end 131 99.5) (width 0.2) (layer "B.Cu") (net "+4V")))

